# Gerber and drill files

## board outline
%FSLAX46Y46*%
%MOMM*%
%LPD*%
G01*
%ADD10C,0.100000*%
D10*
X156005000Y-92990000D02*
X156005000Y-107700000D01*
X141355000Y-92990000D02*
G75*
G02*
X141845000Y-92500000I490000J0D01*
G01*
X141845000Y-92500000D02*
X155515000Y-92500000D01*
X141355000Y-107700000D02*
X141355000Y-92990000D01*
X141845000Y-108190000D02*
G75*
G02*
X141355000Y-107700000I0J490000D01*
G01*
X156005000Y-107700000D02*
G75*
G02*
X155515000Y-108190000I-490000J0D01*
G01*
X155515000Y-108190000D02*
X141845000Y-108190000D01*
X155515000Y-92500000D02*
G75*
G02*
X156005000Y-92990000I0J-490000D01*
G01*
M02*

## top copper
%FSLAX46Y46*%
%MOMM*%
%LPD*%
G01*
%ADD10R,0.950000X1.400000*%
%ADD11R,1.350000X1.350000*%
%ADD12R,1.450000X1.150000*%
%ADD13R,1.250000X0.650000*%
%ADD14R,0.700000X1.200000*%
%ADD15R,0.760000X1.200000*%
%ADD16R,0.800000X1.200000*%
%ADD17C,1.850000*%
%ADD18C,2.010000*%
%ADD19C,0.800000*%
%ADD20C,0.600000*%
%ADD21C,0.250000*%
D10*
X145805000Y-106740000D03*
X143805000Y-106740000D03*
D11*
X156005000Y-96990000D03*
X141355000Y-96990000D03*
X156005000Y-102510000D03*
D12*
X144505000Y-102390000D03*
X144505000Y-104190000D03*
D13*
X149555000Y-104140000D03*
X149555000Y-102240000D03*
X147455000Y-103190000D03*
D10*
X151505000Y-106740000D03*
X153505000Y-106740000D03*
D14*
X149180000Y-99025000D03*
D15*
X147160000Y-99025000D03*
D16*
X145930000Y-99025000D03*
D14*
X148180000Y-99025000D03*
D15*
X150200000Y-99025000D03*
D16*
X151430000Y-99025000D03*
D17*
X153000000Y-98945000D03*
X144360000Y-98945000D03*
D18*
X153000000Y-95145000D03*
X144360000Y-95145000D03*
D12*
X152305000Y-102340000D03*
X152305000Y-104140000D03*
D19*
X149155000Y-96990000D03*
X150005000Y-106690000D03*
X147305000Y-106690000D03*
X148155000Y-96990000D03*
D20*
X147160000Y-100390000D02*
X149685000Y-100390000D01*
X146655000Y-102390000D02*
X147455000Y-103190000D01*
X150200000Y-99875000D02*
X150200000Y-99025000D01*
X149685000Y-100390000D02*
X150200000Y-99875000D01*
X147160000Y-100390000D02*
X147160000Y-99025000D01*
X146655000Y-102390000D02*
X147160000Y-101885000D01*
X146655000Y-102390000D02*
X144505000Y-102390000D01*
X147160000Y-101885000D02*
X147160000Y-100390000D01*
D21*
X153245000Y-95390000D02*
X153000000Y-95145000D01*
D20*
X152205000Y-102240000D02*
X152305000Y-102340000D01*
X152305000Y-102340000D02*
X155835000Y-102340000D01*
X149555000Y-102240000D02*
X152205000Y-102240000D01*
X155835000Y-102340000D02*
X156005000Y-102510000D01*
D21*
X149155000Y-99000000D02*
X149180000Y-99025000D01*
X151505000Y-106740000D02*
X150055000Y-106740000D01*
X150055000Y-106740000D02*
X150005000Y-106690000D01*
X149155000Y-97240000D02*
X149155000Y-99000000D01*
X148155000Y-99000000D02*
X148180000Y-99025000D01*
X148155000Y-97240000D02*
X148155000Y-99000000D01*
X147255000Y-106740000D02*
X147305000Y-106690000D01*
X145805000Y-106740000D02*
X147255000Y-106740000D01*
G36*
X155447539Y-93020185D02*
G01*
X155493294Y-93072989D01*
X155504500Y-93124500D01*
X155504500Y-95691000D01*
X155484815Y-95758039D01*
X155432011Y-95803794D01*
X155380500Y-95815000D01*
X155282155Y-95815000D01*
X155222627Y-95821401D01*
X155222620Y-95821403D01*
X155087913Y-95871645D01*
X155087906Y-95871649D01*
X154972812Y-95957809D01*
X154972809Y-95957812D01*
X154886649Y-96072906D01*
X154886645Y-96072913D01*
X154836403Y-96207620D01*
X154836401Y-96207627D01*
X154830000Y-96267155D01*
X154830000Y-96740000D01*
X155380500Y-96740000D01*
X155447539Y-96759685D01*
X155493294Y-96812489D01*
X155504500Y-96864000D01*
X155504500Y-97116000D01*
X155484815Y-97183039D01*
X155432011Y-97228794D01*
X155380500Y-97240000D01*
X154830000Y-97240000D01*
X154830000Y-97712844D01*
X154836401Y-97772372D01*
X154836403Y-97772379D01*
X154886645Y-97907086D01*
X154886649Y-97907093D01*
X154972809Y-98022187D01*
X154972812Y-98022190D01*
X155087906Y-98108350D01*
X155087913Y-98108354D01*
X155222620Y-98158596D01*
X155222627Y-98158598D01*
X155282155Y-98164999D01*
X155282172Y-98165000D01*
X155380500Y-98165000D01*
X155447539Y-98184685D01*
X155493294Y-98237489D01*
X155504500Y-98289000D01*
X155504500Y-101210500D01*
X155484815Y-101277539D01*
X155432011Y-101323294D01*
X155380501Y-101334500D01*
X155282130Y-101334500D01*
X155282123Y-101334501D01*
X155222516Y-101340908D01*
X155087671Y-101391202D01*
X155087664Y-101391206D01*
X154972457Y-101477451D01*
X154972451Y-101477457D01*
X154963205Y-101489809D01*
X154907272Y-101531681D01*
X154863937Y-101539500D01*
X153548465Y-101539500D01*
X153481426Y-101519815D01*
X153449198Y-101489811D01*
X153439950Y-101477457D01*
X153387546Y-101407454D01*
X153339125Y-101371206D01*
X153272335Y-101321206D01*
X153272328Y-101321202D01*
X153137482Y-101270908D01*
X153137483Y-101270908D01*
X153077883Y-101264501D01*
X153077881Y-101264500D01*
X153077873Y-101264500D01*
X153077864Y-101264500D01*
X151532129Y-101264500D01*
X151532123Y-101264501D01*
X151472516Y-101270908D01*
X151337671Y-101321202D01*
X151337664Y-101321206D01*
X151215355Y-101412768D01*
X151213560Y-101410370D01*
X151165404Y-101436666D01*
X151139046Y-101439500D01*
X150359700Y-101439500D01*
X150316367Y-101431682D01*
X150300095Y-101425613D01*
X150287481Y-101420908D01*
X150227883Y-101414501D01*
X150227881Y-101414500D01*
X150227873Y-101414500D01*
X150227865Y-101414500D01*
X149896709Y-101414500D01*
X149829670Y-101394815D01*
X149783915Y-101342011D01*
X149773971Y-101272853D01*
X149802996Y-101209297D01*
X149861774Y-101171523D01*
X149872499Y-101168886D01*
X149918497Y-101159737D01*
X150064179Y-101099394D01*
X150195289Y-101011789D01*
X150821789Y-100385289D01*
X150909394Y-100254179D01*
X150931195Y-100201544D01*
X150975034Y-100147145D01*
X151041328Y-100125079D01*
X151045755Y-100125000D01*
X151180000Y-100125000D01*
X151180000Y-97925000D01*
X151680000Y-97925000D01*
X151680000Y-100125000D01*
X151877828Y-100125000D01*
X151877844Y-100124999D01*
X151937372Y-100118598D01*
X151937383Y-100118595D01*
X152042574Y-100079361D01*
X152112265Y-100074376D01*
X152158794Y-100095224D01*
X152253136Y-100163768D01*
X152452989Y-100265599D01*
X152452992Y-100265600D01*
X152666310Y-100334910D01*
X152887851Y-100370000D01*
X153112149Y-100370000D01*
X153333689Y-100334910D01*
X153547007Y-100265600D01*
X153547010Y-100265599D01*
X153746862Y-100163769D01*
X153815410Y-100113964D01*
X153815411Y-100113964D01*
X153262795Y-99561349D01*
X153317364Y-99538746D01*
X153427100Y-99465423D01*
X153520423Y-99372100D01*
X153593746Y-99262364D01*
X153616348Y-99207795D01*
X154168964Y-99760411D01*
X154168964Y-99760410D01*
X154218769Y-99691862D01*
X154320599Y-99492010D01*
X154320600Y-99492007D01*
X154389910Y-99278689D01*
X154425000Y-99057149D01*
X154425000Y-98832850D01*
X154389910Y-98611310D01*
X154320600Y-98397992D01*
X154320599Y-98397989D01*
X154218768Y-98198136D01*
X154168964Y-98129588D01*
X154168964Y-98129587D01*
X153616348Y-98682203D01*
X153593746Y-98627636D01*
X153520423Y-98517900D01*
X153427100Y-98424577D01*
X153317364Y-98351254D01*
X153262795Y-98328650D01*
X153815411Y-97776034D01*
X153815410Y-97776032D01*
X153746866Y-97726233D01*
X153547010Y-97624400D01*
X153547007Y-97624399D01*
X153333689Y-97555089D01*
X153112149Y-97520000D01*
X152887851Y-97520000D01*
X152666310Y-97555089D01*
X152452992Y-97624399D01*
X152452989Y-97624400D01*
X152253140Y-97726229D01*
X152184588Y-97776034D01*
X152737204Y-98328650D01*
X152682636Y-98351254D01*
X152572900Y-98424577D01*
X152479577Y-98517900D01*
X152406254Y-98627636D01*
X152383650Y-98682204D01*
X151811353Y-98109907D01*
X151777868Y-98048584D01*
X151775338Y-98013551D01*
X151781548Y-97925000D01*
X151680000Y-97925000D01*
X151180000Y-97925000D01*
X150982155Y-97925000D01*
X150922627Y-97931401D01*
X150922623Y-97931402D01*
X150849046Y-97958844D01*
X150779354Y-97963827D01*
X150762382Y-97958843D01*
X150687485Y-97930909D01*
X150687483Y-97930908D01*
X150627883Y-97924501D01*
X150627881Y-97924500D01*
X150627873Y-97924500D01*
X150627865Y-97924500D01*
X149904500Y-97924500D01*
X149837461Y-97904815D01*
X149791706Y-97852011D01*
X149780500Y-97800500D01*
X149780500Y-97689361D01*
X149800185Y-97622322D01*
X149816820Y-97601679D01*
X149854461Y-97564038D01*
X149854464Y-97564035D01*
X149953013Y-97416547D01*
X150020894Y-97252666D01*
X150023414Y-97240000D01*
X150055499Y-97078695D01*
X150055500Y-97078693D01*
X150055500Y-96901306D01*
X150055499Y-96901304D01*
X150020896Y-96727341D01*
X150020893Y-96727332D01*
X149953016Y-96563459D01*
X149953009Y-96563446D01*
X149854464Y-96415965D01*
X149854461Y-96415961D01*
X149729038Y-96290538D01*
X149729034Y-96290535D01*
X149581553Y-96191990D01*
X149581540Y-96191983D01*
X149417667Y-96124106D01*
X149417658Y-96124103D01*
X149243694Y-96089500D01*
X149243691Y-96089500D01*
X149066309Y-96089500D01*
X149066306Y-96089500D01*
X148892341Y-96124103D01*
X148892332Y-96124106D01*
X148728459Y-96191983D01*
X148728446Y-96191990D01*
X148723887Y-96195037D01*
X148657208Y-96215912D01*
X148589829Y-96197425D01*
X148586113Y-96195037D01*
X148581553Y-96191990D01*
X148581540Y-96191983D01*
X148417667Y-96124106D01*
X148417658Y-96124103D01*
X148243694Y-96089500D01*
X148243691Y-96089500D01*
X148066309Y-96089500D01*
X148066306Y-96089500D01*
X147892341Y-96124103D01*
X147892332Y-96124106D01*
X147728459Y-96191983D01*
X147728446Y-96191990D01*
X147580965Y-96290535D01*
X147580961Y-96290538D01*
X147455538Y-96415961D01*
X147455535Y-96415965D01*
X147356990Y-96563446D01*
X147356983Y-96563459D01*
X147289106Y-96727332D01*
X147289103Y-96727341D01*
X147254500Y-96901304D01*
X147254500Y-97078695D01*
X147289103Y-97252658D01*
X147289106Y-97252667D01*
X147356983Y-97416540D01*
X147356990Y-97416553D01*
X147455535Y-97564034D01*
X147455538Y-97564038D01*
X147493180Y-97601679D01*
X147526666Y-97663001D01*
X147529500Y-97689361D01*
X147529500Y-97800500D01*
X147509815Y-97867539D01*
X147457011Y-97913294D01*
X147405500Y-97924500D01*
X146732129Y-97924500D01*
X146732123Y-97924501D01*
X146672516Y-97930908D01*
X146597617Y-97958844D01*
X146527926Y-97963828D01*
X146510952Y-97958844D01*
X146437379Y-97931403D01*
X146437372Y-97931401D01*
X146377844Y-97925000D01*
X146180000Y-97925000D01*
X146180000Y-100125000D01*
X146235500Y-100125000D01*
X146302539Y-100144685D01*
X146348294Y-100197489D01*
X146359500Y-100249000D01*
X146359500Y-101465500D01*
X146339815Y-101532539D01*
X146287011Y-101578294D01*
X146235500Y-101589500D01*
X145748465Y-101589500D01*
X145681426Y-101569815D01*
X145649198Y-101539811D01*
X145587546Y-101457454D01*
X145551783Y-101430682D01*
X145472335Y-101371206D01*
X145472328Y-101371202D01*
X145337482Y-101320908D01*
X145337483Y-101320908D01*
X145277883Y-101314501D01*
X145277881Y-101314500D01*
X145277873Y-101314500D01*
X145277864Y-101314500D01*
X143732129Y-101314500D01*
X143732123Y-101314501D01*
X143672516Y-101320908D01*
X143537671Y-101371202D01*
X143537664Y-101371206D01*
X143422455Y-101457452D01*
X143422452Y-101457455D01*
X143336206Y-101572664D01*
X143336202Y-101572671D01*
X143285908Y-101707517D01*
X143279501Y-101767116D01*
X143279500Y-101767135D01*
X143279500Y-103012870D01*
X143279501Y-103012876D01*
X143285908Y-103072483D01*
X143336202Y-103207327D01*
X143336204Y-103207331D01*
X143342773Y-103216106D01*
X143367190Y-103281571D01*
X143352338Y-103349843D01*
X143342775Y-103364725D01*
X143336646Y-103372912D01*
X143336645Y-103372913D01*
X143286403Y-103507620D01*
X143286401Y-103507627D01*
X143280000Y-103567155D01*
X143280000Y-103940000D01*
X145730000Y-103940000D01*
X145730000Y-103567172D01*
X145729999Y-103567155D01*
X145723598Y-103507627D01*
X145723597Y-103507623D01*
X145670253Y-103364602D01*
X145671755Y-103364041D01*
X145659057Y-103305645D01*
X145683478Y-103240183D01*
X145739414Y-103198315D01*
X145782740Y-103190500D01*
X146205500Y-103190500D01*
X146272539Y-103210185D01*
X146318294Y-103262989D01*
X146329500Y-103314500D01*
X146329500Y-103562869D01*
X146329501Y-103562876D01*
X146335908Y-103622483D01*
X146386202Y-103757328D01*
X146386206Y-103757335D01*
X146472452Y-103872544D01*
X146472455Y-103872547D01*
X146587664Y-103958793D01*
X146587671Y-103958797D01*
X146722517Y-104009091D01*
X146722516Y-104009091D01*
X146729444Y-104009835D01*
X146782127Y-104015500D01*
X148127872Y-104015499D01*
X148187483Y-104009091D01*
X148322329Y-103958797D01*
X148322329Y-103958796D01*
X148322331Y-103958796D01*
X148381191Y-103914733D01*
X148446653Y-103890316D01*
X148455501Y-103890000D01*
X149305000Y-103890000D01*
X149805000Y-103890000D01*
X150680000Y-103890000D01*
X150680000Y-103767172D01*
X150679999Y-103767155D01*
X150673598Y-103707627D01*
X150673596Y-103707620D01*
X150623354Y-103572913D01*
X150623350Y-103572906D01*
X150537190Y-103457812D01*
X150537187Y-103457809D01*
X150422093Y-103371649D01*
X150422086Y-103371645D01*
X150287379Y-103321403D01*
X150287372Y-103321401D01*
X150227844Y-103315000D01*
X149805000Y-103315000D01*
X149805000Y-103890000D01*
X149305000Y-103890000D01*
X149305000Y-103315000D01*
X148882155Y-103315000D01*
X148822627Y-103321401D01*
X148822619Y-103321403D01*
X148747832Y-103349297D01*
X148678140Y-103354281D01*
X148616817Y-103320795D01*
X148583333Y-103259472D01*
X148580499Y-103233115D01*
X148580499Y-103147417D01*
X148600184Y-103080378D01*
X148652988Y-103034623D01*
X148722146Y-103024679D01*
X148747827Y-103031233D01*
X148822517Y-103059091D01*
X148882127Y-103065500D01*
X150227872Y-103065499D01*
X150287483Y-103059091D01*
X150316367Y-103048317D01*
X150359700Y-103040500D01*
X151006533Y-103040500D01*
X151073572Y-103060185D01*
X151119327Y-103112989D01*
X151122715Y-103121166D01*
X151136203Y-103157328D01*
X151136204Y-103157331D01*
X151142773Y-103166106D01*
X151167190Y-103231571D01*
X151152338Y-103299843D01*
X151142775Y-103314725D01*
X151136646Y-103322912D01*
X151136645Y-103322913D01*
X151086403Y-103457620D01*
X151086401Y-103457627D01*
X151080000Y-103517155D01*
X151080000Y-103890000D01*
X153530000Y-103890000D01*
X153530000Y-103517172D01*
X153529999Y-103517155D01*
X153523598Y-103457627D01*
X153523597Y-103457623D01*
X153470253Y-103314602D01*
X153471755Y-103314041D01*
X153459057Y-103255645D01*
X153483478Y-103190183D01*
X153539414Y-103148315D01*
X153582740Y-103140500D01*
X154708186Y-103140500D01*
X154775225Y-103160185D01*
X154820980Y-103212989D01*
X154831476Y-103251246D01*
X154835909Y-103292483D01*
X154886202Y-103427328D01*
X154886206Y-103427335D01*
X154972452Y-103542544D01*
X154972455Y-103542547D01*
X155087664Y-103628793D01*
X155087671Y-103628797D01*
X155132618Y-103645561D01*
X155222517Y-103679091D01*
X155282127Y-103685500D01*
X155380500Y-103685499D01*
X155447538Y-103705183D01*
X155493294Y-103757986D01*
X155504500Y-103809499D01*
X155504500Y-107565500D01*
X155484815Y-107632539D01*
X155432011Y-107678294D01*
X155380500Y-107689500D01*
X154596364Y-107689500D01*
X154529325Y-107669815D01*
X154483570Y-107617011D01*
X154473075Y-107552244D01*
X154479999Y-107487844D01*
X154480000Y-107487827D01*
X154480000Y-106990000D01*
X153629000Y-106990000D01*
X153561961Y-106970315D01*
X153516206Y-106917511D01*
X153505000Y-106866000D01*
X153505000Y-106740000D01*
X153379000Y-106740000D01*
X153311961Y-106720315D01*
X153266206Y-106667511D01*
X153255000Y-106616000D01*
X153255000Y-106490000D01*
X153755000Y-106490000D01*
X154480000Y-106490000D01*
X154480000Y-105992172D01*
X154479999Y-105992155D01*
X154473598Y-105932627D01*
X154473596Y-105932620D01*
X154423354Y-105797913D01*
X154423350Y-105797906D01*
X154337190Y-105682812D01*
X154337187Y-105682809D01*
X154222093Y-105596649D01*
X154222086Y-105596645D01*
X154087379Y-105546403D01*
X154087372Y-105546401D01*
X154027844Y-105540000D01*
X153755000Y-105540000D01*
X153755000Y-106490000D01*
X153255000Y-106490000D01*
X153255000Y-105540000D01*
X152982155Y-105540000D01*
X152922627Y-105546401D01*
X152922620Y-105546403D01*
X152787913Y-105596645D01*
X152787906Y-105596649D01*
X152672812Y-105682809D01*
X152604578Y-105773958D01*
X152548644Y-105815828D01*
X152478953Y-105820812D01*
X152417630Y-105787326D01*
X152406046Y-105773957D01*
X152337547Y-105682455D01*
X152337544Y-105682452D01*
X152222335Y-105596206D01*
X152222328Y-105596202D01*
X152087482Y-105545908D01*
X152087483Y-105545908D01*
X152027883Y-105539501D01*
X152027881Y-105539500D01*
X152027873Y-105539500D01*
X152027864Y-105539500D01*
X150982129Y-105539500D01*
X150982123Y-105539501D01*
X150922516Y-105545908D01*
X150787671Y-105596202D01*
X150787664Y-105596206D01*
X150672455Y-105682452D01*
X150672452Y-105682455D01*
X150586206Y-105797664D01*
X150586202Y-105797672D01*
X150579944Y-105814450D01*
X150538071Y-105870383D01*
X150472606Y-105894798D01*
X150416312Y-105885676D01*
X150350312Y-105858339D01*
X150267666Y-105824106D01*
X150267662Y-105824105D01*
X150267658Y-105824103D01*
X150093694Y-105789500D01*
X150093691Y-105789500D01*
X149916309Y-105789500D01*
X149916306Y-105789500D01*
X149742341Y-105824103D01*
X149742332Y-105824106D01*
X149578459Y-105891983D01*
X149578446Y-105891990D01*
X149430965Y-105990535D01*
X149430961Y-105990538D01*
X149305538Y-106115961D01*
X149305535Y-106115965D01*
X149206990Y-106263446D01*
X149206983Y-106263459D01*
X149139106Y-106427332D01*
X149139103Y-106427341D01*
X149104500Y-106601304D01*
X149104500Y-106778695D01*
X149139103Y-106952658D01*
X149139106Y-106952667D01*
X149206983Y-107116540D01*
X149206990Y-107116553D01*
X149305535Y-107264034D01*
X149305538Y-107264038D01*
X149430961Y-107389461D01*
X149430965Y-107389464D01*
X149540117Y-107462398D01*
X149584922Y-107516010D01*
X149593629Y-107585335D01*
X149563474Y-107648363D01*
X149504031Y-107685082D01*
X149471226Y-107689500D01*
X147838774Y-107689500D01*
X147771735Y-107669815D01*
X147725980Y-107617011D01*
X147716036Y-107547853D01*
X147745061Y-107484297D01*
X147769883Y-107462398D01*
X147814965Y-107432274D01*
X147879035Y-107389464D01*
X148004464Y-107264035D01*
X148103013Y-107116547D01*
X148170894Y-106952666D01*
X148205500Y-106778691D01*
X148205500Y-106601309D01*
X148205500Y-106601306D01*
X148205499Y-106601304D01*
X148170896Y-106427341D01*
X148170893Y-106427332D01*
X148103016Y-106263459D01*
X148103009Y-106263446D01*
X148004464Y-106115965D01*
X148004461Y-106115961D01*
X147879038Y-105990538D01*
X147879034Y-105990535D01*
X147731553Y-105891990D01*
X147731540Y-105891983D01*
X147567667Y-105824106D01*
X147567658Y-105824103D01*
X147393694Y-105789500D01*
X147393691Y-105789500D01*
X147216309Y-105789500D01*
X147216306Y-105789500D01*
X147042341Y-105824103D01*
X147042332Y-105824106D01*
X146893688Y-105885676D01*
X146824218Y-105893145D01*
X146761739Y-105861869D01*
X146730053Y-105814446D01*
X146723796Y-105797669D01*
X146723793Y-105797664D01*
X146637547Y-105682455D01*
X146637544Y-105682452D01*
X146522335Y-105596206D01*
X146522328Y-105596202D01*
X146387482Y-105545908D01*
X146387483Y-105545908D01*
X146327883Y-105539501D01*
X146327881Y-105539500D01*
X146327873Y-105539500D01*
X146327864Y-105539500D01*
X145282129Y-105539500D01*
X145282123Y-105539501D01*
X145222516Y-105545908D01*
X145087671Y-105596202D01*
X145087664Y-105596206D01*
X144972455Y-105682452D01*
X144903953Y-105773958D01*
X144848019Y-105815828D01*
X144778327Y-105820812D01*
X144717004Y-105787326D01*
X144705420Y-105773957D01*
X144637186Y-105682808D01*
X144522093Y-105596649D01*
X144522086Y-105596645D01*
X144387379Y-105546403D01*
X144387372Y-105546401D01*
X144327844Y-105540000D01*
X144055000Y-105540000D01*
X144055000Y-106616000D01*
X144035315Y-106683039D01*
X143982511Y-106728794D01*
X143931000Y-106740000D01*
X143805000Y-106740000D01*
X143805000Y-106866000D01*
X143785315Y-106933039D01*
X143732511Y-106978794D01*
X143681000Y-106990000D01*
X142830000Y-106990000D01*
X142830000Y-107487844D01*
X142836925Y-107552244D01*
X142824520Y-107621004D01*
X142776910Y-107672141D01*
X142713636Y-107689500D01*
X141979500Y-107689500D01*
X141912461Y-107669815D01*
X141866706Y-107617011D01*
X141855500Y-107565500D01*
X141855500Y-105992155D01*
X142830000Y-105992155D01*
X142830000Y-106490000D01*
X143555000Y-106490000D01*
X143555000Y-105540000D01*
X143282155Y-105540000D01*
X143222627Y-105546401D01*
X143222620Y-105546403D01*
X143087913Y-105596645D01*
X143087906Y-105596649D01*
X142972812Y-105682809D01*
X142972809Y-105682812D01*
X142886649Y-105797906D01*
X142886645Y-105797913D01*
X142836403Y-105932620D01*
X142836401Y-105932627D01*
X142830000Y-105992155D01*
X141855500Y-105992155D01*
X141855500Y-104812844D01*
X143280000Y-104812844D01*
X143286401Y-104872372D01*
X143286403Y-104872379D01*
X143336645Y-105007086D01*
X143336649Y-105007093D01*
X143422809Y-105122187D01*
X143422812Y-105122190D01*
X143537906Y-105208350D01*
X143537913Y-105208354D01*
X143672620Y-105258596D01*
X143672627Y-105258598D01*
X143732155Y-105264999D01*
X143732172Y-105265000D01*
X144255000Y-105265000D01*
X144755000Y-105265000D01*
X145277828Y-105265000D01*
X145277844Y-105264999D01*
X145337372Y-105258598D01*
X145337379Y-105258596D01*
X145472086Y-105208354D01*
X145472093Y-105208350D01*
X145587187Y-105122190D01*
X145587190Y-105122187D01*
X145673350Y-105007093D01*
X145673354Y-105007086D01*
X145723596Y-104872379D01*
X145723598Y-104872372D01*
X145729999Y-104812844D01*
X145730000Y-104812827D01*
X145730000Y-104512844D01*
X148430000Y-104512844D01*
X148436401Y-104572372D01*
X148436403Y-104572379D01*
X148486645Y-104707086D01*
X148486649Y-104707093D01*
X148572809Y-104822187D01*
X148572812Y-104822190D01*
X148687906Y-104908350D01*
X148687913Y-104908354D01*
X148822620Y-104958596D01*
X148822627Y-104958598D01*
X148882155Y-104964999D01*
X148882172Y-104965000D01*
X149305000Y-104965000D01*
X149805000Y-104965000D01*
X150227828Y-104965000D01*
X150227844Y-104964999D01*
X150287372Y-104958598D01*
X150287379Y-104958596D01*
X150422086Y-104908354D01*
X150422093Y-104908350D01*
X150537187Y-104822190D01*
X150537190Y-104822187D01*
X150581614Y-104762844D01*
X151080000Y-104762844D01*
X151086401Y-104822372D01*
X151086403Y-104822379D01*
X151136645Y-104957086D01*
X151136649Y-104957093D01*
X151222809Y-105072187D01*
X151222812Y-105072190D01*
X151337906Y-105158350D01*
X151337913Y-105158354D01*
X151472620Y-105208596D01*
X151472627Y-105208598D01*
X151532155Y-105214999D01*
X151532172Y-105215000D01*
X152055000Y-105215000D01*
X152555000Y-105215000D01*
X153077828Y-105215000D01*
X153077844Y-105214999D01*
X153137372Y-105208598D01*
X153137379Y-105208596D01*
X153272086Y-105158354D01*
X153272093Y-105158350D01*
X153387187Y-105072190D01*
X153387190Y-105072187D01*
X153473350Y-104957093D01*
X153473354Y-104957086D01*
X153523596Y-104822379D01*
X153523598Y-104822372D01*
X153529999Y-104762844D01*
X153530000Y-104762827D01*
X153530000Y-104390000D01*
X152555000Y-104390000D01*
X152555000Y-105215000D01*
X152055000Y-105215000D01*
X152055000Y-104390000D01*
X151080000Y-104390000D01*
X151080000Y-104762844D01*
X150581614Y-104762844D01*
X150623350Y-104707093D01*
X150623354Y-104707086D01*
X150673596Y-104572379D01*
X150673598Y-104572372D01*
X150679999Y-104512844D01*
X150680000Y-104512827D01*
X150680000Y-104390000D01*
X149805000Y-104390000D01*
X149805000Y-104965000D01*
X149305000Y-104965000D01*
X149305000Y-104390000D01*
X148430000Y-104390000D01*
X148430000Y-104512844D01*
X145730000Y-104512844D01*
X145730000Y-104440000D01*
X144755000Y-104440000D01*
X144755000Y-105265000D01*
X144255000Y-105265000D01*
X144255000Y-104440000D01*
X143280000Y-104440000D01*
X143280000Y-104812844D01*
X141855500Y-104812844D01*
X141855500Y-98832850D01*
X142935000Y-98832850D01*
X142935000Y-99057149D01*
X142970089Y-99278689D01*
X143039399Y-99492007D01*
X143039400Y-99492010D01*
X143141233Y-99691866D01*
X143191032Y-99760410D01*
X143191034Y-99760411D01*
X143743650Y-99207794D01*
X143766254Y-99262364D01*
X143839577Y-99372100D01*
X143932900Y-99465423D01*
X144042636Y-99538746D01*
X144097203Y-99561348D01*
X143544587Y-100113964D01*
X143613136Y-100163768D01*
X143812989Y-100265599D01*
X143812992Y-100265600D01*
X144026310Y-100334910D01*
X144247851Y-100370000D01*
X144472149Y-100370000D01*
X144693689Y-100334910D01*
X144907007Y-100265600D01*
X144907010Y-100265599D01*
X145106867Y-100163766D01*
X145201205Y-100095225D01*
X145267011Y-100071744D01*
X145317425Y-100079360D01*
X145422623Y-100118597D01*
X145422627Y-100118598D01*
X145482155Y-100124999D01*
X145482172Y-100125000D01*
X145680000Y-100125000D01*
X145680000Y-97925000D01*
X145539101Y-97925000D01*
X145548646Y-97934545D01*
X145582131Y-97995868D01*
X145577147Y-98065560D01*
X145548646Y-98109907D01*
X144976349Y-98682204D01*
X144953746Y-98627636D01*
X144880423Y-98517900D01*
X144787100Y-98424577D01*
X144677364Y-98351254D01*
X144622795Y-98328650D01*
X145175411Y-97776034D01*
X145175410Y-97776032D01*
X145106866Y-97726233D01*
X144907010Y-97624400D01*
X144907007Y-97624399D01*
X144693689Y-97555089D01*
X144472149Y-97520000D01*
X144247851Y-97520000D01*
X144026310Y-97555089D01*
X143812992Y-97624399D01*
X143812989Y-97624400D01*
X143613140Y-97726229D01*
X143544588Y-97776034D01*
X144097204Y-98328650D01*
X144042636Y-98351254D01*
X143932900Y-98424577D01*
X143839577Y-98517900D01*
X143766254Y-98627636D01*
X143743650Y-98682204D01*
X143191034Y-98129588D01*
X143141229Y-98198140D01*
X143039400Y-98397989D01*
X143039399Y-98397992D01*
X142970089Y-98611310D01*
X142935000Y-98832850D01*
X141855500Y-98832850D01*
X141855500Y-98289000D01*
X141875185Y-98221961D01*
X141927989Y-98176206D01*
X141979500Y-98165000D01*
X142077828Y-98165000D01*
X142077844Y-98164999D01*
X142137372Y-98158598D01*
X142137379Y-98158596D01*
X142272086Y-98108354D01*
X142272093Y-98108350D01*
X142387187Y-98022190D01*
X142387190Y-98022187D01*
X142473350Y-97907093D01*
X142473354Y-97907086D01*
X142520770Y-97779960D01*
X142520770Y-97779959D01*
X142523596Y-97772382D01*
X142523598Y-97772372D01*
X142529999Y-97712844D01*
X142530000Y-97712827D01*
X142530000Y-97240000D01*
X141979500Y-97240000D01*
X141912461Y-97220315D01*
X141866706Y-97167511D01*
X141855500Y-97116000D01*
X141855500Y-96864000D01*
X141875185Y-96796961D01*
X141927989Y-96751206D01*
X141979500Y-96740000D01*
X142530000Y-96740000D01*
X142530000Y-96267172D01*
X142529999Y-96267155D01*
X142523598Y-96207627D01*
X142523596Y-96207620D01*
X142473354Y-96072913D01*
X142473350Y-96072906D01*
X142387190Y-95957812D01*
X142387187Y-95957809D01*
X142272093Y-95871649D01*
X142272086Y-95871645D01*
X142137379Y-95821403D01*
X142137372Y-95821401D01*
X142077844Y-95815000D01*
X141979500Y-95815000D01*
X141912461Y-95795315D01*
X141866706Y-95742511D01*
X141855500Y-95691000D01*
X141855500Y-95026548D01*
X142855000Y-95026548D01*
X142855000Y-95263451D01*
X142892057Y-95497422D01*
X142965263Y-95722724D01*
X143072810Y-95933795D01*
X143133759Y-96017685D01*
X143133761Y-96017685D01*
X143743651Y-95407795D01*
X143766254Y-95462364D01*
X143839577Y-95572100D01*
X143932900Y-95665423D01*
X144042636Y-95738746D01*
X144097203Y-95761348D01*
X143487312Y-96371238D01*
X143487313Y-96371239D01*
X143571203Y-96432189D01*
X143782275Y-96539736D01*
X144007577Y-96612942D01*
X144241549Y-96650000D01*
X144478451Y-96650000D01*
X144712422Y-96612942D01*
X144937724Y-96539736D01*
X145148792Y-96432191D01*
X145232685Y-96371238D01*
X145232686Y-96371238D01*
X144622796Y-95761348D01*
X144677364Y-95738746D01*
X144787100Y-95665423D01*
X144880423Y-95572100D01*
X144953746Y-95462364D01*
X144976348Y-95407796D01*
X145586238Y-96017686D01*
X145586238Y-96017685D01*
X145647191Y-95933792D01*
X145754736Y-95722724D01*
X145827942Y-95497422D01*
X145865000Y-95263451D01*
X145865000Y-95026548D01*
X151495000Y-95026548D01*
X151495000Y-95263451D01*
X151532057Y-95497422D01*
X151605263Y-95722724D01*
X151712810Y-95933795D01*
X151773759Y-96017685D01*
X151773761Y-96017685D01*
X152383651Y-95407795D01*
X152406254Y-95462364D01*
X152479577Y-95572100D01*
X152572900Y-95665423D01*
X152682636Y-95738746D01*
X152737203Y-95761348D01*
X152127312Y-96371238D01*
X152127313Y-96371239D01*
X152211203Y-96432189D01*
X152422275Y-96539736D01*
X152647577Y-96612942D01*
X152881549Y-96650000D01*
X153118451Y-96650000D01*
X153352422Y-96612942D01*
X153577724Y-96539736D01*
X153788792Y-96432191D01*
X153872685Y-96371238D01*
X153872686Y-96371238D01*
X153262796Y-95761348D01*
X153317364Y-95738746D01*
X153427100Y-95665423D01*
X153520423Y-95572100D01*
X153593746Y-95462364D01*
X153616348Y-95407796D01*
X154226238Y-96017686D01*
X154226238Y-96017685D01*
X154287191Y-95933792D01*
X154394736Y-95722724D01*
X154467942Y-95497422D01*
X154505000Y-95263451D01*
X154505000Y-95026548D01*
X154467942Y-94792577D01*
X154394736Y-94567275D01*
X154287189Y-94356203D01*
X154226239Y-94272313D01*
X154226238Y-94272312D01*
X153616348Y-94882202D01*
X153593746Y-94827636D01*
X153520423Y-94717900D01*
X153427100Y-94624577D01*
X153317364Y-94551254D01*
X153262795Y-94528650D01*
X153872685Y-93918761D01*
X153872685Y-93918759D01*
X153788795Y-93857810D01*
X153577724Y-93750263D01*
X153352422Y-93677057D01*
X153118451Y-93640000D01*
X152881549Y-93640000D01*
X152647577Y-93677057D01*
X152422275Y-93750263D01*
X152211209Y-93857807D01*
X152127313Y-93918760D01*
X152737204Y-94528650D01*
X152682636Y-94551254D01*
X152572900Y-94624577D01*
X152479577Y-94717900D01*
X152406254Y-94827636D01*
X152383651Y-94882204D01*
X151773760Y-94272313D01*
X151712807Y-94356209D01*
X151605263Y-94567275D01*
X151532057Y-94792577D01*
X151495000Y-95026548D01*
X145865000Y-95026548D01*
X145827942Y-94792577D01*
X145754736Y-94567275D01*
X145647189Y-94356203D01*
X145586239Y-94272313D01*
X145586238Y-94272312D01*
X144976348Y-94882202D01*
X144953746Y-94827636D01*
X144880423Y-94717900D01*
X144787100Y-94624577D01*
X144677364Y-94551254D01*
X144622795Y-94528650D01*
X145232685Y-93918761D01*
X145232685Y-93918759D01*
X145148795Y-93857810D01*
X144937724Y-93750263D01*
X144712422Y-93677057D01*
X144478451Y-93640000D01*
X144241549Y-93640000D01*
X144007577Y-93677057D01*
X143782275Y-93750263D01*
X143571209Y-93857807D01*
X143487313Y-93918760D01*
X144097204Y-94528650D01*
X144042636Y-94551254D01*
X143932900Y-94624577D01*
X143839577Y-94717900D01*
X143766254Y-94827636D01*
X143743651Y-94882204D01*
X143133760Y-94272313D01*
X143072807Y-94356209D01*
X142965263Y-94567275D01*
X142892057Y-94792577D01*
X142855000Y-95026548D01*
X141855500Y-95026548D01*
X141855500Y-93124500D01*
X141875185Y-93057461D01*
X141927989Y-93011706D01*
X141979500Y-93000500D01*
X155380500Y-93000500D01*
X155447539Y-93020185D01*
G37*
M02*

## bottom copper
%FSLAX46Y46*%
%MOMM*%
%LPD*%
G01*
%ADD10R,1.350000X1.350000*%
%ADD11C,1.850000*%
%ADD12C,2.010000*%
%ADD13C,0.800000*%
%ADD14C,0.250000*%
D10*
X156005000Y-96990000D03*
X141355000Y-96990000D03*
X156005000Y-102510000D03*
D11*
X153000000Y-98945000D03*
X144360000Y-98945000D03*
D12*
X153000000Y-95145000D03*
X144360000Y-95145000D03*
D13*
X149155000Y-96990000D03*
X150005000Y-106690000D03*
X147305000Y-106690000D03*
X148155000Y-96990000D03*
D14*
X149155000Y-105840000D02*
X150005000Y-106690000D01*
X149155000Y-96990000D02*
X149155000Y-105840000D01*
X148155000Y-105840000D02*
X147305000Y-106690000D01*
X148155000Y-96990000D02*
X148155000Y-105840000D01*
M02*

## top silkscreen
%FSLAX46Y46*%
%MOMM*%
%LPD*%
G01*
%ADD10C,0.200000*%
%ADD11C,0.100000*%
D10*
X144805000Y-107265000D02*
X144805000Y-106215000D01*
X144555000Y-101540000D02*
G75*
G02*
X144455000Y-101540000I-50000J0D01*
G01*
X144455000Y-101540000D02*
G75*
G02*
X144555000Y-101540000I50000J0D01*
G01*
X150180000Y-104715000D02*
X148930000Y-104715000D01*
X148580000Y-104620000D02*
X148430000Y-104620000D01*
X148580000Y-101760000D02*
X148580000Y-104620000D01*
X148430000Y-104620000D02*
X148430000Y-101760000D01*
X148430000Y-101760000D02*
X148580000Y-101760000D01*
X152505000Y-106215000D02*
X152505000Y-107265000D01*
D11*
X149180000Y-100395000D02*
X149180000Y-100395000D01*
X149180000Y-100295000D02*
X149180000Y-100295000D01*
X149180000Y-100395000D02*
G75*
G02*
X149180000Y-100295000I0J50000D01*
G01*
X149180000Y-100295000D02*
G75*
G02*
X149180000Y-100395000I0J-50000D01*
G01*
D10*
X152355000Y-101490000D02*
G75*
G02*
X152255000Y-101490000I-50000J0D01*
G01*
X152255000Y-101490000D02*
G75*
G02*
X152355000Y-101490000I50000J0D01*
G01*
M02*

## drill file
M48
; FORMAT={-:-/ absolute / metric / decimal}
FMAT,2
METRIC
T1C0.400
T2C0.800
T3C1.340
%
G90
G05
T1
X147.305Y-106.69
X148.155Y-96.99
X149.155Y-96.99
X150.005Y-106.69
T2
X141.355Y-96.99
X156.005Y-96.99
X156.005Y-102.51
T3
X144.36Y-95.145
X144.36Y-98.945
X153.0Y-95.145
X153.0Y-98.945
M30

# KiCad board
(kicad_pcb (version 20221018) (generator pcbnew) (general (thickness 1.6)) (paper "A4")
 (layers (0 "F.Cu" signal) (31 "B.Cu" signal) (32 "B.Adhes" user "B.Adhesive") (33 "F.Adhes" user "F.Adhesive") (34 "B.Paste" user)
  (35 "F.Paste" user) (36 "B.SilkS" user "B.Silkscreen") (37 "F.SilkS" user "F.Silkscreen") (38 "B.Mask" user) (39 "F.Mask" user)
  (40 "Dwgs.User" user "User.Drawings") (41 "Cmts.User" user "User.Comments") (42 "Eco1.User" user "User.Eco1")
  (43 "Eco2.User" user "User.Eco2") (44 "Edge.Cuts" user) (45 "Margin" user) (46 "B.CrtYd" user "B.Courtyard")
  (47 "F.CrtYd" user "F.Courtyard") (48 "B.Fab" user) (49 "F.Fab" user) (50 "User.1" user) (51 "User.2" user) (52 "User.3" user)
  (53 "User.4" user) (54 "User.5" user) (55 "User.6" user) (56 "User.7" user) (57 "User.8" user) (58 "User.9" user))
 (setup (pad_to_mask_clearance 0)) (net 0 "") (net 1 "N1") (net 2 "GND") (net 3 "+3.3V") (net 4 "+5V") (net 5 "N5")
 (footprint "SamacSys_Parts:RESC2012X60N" (layer "F.Cu") (at 144.805 106.74 180)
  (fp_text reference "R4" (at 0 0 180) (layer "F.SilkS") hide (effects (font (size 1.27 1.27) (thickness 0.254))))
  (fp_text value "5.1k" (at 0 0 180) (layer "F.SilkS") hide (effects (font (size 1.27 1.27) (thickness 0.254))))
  (fp_line (start 0 -0.525) (end 0 0.525) (stroke (width 0.2) (type solid)) (layer "F.SilkS"))
  (pad "1" smd rect (at -1 0 180) (size 0.95 1.4) (layers "F.Cu" "F.Paste" "F.Mask") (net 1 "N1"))
  (pad "2" smd rect (at 1 0 180) (size 0.95 1.4) (layers "F.Cu" "F.Paste" "F.Mask") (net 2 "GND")))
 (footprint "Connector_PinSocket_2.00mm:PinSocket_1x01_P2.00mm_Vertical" (layer "F.Cu") (at 156.005 96.99)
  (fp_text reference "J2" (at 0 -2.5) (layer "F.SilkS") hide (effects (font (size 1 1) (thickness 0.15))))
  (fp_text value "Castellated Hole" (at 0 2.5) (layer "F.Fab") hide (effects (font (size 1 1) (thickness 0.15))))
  (pad "1" thru_hole rect (at 0 0) (size 1.35 1.35) (drill 0.8) (layers "*.Cu" "*.Mask") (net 2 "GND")))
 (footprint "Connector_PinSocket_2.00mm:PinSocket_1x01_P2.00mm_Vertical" (layer "F.Cu") (at 141.355 96.99)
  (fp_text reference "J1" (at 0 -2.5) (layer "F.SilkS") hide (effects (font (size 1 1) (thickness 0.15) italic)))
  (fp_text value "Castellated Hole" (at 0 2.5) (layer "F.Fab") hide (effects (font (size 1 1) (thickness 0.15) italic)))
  (pad "1" thru_hole rect (at 0 0) (size 1.35 1.35) (drill 0.8) (layers "*.Cu" "*.Mask") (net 2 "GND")))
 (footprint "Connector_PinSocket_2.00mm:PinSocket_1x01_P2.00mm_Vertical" (layer "F.Cu") (at 156.005 102.51 180)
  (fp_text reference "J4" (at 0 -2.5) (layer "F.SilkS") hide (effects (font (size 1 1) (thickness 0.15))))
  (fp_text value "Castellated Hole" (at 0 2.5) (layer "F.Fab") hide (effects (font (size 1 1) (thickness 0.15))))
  (pad "1" thru_hole rect (at 0 0 180) (size 1.35 1.35) (drill 0.8) (layers "*.Cu" "*.Mask") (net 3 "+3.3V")))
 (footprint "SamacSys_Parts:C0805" (layer "F.Cu") (at 144.505 103.29 -90)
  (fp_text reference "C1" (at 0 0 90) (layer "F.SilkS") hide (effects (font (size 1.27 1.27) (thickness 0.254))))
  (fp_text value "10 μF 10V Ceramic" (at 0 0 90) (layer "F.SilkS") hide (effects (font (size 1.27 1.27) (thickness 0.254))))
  (fp_circle (center -1.75 0) (end -1.75 0.05) (stroke (width 0.2) (type solid)) (fill none) (layer "F.SilkS"))
  (pad "1" smd rect (at -0.9 0 270) (size 1.15 1.45) (layers "F.Cu" "F.Paste" "F.Mask") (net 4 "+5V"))
  (pad "2" smd rect (at 0.9 0 270) (size 1.15 1.45) (layers "F.Cu" "F.Paste" "F.Mask") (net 2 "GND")))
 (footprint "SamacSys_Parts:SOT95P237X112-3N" (layer "F.Cu") (at 148.505 103.19 180)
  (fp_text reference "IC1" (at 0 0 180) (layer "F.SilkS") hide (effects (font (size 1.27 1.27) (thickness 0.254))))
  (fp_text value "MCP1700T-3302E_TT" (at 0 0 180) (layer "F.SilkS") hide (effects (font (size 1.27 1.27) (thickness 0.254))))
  (fp_line (start -1.675 -1.525) (end -0.425 -1.525) (stroke (width 0.2) (type solid)) (layer "F.SilkS"))
  (fp_line (start -0.075 -1.43) (end 0.075 -1.43) (stroke (width 0.2) (type solid)) (layer "F.SilkS"))
  (fp_line (start -0.075 1.43) (end -0.075 -1.43) (stroke (width 0.2) (type solid)) (layer "F.SilkS"))
  (fp_line (start 0.075 -1.43) (end 0.075 1.43) (stroke (width 0.2) (type solid)) (layer "F.SilkS"))
  (fp_line (start 0.075 1.43) (end -0.075 1.43) (stroke (width 0.2) (type solid)) (layer "F.SilkS"))
  (pad "1" smd rect (at -1.05 -0.95 270) (size 0.65 1.25) (layers "F.Cu" "F.Paste" "F.Mask") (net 2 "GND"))
  (pad "2" smd rect (at -1.05 0.95 270) (size 0.65 1.25) (layers "F.Cu" "F.Paste" "F.Mask") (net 3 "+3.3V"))
  (pad "3" smd rect (at 1.05 0 270) (size 0.65 1.25) (layers "F.Cu" "F.Paste" "F.Mask") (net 4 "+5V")))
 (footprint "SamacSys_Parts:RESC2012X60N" (layer "F.Cu") (at 152.505 106.74)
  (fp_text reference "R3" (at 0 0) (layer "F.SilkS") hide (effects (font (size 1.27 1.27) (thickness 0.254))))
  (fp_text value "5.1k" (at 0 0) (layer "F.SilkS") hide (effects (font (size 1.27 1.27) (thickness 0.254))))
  (fp_line (start 0 -0.525) (end 0 0.525) (stroke (width 0.2) (type solid)) (layer "F.SilkS"))
  (pad "1" smd rect (at -1 0) (size 0.95 1.4) (layers "F.Cu" "F.Paste" "F.Mask") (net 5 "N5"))
  (pad "2" smd rect (at 1 0) (size 0.95 1.4) (layers "F.Cu" "F.Paste" "F.Mask") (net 2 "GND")))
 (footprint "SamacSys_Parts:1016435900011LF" (layer "F.Cu") (at 148.68 95.995 180)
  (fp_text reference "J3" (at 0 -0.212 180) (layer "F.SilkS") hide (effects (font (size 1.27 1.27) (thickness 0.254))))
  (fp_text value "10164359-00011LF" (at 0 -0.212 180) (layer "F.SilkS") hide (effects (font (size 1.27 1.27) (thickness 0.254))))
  (fp_line (start -0.5 -4.4) (end -0.5 -4.4) (stroke (width 0.1) (type solid)) (layer "F.SilkS"))
  (fp_line (start -0.5 -4.3) (end -0.5 -4.3) (stroke (width 0.1) (type solid)) (layer "F.SilkS"))
  (fp_arc (start -0.5 -4.4) (mid -0.45 -4.35) (end -0.5 -4.3) (stroke (width 0.1) (type solid)) (layer "F.SilkS"))
  (fp_arc (start -0.5 -4.3) (mid -0.55 -4.35) (end -0.5 -4.4) (stroke (width 0.1) (type solid)) (layer "F.SilkS"))
  (pad "A5" smd rect (at -0.5 -3.03 180) (size 0.7 1.2) (layers "F.Cu" "F.Paste" "F.Mask") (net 5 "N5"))
  (pad "A9" smd rect (at 1.52 -3.03 180) (size 0.76 1.2) (layers "F.Cu" "F.Paste" "F.Mask") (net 4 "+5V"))
  (pad "A12" smd rect (at 2.75 -3.03 180) (size 0.8 1.2) (layers "F.Cu" "F.Paste" "F.Mask") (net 2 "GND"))
  (pad "B5" smd rect (at 0.5 -3.03 180) (size 0.7 1.2) (layers "F.Cu" "F.Paste" "F.Mask") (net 1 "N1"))
  (pad "B9" smd rect (at -1.52 -3.03 180) (size 0.76 1.2) (layers "F.Cu" "F.Paste" "F.Mask") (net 4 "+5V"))
  (pad "B12" smd rect (at -2.75 -3.03 180) (size 0.8 1.2) (layers "F.Cu" "F.Paste" "F.Mask") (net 2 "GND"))
  (pad "MH1" thru_hole circle (at -4.32 -2.95 180) (size 1.85 1.85) (drill 1.34) (layers "*.Cu" "*.Mask") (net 2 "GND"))
  (pad "MH2" thru_hole circle (at 4.32 -2.95 180) (size 1.85 1.85) (drill 1.34) (layers "*.Cu" "*.Mask") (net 2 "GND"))
  (pad "MH3" thru_hole circle (at -4.32 0.85 180) (size 2.01 2.01) (drill 1.34) (layers "*.Cu" "*.Mask") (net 2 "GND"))
  (pad "MH4" thru_hole circle (at 4.32 0.85 180) (size 2.01 2.01) (drill 1.34) (layers "*.Cu" "*.Mask") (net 2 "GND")))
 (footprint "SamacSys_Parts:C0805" (layer "F.Cu") (at 152.305 103.24 -90)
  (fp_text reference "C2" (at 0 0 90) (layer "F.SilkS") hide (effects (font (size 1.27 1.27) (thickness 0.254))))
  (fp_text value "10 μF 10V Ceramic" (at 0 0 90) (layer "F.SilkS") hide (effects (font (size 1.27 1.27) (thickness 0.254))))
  (fp_circle (center -1.75 0) (end -1.75 0.05) (stroke (width 0.2) (type solid)) (fill none) (layer "F.SilkS"))
  (pad "1" smd rect (at -0.9 0 270) (size 1.15 1.45) (layers "F.Cu" "F.Paste" "F.Mask") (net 3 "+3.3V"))
  (pad "2" smd rect (at 0.9 0 270) (size 1.15 1.45) (layers "F.Cu" "F.Paste" "F.Mask") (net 2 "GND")))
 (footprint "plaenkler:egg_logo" (layer "B.Cu") (at 146.305 103.49 90)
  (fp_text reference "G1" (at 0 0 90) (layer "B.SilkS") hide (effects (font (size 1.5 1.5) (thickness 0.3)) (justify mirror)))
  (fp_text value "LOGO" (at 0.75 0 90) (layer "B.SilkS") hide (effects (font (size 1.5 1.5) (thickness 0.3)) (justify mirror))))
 (gr_line (start 156.005 92.99) (end 156.005 107.7) (stroke (width 0.1) (type default)) (layer "Edge.Cuts"))
 (gr_arc (start 141.355 92.99) (mid 141.498518 92.643518) (end 141.845 92.5) (stroke (width 0.1) (type default)) (layer "Edge.Cuts"))
 (gr_line (start 141.845 92.5) (end 155.515 92.5) (stroke (width 0.1) (type default)) (layer "Edge.Cuts"))
 (gr_line (start 141.355 107.7) (end 141.355 92.99) (stroke (width 0.1) (type default)) (layer "Edge.Cuts"))
 (gr_arc (start 141.845 108.19) (mid 141.498518 108.046482) (end 141.355 107.7) (stroke (width 0.1) (type default)) (layer "Edge.Cuts"))
 (gr_arc (start 156.005 107.7) (mid 155.861482 108.046482) (end 155.515 108.19) (stroke (width 0.1) (type default)) (layer "Edge.Cuts"))
 (gr_line (start 155.515 108.19) (end 141.845 108.19) (stroke (width 0.1) (type default)) (layer "Edge.Cuts"))
 (gr_arc (start 155.515 92.5) (mid 155.861482 92.643518) (end 156.005 92.99) (stroke (width 0.1) (type default)) (layer "Edge.Cuts"))
 (segment (start 147.16 100.39) (end 149.685 100.39) (width 0.6) (layer "F.Cu") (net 4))
 (segment (start 146.655 102.39) (end 147.455 103.19) (width 0.6) (layer "F.Cu") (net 4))
 (segment (start 150.2 99.875) (end 150.2 99.025) (width 0.6) (layer "F.Cu") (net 4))
 (segment (start 149.685 100.39) (end 150.2 99.875) (width 0.6) (layer "F.Cu") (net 4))
 (segment (start 147.16 100.39) (end 147.16 99.025) (width 0.6) (layer "F.Cu") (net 4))
 (segment (start 146.655 102.39) (end 147.16 101.885) (width 0.6) (layer "F.Cu") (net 4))
 (segment (start 146.655 102.39) (end 144.505 102.39) (width 0.6) (layer "F.Cu") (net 4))
 (segment (start 147.16 101.885) (end 147.16 100.39) (width 0.6) (layer "F.Cu") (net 4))
 (segment (start 153.245 95.39) (end 153 95.145) (width 0.25) (layer "F.Cu") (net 2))
 (segment (start 152.205 102.24) (end 152.305 102.34) (width 0.6) (layer "F.Cu") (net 3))
 (segment (start 152.305 102.34) (end 155.835 102.34) (width 0.6) (layer "F.Cu") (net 3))
 (segment (start 149.555 102.24) (end 152.205 102.24) (width 0.6) (layer "F.Cu") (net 3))
 (segment (start 155.835 102.34) (end 156.005 102.51) (width 0.6) (layer "F.Cu") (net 3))
 (segment (start 149.155 99) (end 149.18 99.025) (width 0.25) (layer "F.Cu") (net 5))
 (segment (start 151.505 106.74) (end 150.055 106.74) (width 0.25) (layer "F.Cu") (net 5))
 (segment (start 150.055 106.74) (end 150.005 106.69) (width 0.25) (layer "F.Cu") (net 5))
 (segment (start 149.155 97.24) (end 149.155 99) (width 0.25) (layer "F.Cu") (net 5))
 (via (at 149.155 96.99) (size 0.8) (drill 0.4) (layers "F.Cu" "B.Cu") (free) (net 5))
 (via (at 150.005 106.69) (size 0.8) (drill 0.4) (layers "F.Cu" "B.Cu") (free) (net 5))
 (segment (start 149.155 105.84) (end 150.005 106.69) (width 0.25) (layer "B.Cu") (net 5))
 (segment (start 149.155 96.99) (end 149.155 105.84) (width 0.25) (layer "B.Cu") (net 5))
 (segment (start 148.155 99) (end 148.18 99.025) (width 0.25) (layer "F.Cu") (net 1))
 (segment (start 148.155 97.24) (end 148.155 99) (width 0.25) (layer "F.Cu") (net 1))
 (segment (start 147.255 106.74) (end 147.305 106.69) (width 0.25) (layer "F.Cu") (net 1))
 (segment (start 145.805 106.74) (end 147.255 106.74) (width 0.25) (layer "F.Cu") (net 1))
 (via (at 147.305 106.69) (size 0.8) (drill 0.4) (layers "F.Cu" "B.Cu") (free) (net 1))
 (via (at 148.155 96.99) (size 0.8) (drill 0.4) (layers "F.Cu" "B.Cu") (free) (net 1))
 (segment (start 148.155 105.84) (end 147.305 106.69) (width 0.25) (layer "B.Cu") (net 1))
 (segment (start 148.155 96.99) (end 148.155 105.84) (width 0.25) (layer "B.Cu") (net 1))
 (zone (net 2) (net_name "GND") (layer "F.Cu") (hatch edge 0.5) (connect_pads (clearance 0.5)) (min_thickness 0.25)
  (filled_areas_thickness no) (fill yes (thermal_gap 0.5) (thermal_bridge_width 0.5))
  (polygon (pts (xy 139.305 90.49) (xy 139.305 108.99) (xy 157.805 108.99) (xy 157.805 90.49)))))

